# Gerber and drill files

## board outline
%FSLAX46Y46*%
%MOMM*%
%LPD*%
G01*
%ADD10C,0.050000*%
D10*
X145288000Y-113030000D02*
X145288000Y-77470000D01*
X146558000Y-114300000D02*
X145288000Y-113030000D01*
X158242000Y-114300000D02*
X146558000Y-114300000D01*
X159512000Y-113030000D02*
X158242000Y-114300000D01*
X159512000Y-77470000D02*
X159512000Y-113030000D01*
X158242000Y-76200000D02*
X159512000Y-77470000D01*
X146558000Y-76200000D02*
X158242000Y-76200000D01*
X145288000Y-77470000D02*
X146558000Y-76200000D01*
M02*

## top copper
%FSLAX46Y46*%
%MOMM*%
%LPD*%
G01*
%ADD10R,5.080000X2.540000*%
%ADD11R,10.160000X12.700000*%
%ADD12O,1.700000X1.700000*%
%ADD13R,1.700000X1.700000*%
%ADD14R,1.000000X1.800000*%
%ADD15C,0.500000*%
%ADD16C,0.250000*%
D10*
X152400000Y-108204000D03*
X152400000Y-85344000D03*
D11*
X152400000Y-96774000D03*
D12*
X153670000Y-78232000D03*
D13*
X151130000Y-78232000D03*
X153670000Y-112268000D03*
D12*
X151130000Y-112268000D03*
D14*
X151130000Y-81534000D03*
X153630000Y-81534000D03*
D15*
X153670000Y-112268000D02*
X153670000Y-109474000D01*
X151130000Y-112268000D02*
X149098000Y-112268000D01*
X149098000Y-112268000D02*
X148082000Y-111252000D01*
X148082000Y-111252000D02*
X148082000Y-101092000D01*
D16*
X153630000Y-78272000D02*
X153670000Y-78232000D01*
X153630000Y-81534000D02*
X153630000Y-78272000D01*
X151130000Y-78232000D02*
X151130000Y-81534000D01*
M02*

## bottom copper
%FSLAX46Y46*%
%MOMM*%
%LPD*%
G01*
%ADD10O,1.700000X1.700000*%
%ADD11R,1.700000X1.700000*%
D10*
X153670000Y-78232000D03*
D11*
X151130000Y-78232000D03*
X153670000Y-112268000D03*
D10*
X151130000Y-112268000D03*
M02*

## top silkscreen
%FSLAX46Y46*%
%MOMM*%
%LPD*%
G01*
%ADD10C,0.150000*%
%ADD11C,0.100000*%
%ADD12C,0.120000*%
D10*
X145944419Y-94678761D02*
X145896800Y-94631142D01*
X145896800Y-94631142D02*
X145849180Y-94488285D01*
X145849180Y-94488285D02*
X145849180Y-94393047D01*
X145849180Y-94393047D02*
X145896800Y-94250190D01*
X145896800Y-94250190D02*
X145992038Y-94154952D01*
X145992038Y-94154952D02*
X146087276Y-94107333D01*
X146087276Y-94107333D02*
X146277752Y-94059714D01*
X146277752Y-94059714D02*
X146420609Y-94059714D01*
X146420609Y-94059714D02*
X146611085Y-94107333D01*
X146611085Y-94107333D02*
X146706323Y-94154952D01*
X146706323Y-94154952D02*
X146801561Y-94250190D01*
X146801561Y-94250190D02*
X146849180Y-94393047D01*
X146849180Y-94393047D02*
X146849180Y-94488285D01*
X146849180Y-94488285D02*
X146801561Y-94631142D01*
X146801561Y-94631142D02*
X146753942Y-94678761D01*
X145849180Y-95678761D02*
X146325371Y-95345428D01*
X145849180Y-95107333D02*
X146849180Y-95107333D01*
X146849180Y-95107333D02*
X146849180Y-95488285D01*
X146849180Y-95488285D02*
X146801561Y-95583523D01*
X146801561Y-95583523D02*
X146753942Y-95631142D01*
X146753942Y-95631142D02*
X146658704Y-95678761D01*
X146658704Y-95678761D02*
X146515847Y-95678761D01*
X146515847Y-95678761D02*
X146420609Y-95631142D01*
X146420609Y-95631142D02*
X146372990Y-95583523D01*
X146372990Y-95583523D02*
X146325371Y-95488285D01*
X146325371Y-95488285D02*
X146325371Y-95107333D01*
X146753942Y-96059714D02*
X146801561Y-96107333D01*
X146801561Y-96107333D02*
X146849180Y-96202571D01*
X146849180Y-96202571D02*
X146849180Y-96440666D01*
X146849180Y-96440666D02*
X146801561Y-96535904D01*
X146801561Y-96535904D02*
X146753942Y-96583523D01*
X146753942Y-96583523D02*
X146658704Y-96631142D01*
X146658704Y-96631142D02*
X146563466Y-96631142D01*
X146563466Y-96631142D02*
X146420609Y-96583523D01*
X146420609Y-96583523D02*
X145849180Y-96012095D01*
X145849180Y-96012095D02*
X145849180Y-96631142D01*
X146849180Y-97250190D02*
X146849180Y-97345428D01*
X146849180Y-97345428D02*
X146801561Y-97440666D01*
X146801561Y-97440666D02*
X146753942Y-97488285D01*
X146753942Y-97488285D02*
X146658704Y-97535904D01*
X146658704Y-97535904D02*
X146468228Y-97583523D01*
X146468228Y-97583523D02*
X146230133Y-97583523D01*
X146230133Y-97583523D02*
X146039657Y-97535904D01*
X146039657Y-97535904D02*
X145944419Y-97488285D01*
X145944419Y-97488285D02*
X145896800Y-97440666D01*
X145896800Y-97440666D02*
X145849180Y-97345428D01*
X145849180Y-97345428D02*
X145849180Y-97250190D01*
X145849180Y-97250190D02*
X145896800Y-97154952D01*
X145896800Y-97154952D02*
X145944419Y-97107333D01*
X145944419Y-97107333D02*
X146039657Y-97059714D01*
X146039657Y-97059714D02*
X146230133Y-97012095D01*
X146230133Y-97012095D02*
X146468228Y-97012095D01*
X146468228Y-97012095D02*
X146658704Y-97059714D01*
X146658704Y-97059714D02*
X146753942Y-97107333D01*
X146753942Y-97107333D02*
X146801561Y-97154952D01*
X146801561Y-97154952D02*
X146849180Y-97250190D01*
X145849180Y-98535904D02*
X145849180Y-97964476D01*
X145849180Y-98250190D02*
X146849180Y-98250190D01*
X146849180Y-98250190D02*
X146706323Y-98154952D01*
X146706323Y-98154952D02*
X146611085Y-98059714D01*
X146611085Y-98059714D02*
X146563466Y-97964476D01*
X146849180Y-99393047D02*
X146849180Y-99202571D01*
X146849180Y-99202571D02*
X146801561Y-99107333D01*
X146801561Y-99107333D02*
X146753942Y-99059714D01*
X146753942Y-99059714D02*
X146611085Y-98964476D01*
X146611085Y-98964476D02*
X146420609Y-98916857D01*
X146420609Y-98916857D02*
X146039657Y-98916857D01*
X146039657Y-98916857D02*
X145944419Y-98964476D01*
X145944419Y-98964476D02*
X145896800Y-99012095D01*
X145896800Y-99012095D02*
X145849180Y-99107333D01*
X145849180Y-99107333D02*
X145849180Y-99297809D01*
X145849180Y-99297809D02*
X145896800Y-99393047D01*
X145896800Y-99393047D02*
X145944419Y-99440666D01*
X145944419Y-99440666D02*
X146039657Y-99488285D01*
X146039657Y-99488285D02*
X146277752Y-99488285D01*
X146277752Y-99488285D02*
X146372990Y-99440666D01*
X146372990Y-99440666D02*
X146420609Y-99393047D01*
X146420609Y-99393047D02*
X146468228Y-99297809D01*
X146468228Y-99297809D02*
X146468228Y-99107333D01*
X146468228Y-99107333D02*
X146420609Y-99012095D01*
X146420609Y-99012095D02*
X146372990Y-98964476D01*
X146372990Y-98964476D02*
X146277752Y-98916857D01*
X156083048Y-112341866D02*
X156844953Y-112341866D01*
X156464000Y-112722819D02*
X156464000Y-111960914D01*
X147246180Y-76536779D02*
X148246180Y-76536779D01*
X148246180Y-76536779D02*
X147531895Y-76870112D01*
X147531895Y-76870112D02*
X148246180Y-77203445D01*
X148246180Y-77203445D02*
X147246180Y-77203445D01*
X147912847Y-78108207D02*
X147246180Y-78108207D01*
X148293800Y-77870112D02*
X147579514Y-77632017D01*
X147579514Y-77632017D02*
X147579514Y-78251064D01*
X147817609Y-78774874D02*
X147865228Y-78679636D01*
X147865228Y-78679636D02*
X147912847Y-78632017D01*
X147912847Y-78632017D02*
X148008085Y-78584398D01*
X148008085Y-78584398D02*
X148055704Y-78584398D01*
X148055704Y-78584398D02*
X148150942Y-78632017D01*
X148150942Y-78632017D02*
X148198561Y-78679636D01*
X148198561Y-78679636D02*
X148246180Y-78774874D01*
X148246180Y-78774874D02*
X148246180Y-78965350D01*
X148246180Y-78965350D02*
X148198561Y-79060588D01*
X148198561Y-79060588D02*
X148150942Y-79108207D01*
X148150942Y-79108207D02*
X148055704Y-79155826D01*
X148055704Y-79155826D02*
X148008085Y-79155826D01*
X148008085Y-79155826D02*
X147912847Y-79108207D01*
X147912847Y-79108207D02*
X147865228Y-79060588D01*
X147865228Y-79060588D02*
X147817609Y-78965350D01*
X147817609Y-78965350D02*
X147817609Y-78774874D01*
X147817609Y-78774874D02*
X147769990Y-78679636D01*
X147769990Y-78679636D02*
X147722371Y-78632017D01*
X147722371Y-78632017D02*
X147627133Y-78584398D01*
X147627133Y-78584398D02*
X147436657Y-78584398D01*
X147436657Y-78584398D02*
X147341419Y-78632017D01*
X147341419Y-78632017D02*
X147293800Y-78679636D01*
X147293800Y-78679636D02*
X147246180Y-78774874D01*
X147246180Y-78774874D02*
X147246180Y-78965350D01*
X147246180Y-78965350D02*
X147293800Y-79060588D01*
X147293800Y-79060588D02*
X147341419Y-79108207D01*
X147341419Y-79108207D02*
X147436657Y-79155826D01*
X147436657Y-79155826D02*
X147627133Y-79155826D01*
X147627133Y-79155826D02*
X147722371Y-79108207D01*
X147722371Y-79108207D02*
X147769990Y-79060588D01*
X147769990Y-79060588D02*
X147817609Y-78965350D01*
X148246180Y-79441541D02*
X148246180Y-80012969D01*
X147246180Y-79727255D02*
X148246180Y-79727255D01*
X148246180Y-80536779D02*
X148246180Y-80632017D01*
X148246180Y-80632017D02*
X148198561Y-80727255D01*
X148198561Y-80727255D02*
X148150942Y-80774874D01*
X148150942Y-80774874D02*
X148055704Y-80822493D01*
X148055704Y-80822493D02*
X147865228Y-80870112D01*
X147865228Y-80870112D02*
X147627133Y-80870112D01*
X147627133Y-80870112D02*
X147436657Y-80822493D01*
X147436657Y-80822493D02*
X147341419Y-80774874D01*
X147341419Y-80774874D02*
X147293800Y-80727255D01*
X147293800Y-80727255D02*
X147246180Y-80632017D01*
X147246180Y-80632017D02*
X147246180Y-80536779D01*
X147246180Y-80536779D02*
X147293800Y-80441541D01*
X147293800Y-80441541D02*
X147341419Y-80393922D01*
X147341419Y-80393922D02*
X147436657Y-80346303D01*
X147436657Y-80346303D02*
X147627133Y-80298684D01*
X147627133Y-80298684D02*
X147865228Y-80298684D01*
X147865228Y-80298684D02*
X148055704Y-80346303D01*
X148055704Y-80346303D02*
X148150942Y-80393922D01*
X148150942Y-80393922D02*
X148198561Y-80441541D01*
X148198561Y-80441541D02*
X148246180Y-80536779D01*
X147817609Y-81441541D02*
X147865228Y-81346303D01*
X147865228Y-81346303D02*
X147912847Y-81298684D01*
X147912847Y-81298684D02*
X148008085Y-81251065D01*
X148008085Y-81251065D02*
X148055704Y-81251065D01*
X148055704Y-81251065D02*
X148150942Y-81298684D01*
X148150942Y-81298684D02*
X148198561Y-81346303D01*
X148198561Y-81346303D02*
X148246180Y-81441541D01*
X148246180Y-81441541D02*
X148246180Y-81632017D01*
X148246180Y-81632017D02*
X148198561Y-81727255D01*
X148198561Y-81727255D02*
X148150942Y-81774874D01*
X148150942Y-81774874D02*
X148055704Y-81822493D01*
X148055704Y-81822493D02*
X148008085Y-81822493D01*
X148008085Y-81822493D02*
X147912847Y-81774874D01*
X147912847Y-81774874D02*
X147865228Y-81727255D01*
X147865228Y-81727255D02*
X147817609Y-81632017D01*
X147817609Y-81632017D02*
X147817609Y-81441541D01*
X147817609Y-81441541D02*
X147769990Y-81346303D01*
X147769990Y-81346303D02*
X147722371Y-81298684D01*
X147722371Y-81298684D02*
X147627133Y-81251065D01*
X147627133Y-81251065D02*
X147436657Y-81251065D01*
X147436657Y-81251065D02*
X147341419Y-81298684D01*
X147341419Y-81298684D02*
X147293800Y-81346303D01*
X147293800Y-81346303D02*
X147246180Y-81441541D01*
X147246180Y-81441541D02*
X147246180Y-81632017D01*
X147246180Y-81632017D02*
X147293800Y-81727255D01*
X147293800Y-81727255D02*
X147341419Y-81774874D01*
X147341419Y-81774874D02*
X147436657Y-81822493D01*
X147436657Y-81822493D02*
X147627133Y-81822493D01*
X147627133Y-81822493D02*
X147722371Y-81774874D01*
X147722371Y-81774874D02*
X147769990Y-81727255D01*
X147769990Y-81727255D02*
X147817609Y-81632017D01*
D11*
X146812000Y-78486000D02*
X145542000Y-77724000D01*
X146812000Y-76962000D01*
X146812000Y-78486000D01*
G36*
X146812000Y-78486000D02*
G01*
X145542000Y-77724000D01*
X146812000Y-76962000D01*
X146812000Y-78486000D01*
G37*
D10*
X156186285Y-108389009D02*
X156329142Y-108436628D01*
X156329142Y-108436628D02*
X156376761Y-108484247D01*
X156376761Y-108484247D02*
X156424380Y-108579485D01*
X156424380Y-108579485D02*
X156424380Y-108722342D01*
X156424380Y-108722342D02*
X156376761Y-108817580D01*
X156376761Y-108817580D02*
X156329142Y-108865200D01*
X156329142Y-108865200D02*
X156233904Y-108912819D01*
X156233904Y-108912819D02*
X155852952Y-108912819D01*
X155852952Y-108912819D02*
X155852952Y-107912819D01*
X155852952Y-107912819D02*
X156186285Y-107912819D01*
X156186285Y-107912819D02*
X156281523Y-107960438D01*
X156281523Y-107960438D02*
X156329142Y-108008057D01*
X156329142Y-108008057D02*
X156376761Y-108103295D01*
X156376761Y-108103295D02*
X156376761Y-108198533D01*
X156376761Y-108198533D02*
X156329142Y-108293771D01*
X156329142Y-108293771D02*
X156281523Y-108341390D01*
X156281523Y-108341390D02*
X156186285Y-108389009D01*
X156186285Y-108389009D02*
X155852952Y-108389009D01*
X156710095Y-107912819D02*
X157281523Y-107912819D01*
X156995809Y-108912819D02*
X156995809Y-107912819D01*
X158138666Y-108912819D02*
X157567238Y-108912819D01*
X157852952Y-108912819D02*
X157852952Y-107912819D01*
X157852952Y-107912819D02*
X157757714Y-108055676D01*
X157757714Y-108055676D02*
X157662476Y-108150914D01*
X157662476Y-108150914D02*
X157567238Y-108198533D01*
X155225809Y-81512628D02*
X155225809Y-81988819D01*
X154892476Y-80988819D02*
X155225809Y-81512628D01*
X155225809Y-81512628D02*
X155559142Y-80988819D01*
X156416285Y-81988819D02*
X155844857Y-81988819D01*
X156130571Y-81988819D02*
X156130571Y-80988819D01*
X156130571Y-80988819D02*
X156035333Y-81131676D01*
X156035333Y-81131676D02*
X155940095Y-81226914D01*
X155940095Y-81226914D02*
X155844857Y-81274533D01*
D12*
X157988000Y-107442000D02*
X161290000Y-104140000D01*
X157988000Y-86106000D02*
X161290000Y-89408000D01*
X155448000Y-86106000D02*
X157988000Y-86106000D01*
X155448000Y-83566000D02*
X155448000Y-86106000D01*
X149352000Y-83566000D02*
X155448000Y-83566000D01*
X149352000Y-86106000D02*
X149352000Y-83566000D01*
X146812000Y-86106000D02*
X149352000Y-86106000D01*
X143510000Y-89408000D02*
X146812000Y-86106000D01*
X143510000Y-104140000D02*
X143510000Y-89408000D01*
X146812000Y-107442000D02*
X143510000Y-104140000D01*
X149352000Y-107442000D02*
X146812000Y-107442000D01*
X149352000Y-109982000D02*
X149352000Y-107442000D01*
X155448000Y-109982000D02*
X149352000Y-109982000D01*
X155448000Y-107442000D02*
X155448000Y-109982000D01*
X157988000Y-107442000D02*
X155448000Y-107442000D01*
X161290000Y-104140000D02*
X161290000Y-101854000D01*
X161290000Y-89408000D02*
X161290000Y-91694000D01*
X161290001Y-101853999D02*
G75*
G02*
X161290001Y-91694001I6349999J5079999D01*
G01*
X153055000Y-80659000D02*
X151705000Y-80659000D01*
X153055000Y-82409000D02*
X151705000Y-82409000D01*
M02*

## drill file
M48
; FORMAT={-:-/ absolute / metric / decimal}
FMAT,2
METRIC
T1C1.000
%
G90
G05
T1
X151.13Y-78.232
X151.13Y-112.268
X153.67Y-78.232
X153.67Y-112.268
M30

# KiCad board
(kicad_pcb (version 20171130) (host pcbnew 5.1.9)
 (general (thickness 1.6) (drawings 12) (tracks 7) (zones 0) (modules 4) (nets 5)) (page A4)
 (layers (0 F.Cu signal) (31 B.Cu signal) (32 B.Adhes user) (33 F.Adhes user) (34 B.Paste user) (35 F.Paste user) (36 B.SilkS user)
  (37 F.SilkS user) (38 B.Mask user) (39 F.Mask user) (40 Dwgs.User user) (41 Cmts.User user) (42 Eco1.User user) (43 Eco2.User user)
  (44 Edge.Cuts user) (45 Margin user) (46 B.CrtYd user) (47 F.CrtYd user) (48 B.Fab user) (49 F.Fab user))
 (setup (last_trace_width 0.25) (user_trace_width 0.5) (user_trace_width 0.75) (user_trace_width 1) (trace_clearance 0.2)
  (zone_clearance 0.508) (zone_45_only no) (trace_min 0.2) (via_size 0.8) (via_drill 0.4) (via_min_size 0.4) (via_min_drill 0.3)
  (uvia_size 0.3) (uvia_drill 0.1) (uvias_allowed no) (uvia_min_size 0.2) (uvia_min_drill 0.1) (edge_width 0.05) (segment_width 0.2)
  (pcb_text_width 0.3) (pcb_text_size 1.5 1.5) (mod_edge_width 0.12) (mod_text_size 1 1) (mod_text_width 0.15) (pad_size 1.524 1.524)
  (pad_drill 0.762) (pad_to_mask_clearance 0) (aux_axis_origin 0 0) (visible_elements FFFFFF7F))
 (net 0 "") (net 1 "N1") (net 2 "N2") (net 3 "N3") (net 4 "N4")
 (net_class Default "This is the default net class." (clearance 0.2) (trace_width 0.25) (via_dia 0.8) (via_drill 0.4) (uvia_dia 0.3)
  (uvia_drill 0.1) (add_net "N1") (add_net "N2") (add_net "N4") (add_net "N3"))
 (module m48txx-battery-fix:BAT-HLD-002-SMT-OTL (layer F.Cu) (at 152.4 96.774 90)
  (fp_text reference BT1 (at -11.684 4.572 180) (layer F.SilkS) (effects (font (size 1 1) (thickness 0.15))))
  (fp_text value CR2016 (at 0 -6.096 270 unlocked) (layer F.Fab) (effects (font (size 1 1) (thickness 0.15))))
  (fp_line (start -10.668 5.588) (end -7.366 8.89) (layer F.SilkS) (width 0.12))
  (fp_line (start 10.668 5.588) (end 7.366 8.89) (layer F.SilkS) (width 0.12))
  (fp_line (start 10.668 3.048) (end 10.668 5.588) (layer F.SilkS) (width 0.12))
  (fp_line (start 13.208 3.048) (end 10.668 3.048) (layer F.SilkS) (width 0.12))
  (fp_line (start 13.208 -3.048) (end 13.208 3.048) (layer F.SilkS) (width 0.12))
  (fp_line (start 10.668 -3.048) (end 13.208 -3.048) (layer F.SilkS) (width 0.12))
  (fp_line (start 10.668 -5.588) (end 10.668 -3.048) (layer F.SilkS) (width 0.12))
  (fp_line (start 7.366 -8.89) (end 10.668 -5.588) (layer F.SilkS) (width 0.12))
  (fp_line (start -7.366 -8.89) (end 7.366 -8.89) (layer F.SilkS) (width 0.12))
  (fp_line (start -10.668 -5.588) (end -7.366 -8.89) (layer F.SilkS) (width 0.12))
  (fp_line (start -10.668 -3.048) (end -10.668 -5.588) (layer F.SilkS) (width 0.12))
  (fp_line (start -13.208 -3.048) (end -10.668 -3.048) (layer F.SilkS) (width 0.12))
  (fp_line (start -13.208 3.048) (end -13.208 -3.048) (layer F.SilkS) (width 0.12))
  (fp_line (start -10.668 3.048) (end -13.208 3.048) (layer F.SilkS) (width 0.12))
  (fp_line (start -10.668 5.588) (end -10.668 3.048) (layer F.SilkS) (width 0.12))
  (fp_line (start -7.366 8.89) (end -5.08 8.89) (layer F.SilkS) (width 0.12))
  (fp_line (start 7.366 8.89) (end 5.08 8.89) (layer F.SilkS) (width 0.12))
  (fp_arc (start 0 15.24) (end 5.079999 8.890001) (angle -77.31961651) (layer F.SilkS) (width 0.12))
  (pad 1 smd rect (at -12.7 0 90) (size 2.54 5.08) (drill (offset 1.27 0)) (layers F.Cu F.Paste F.Mask) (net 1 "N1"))
  (pad 1 smd rect (at 12.7 0 90) (size 2.54 5.08) (drill (offset -1.27 0)) (layers F.Cu F.Paste F.Mask) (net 1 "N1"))
  (pad 2 smd rect (at 0 0 90) (size 12.7 10.16) (layers F.Cu F.Mask) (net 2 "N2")))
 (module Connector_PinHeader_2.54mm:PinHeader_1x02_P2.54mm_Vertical (layer B.Cu) (at 151.13 78.232 270)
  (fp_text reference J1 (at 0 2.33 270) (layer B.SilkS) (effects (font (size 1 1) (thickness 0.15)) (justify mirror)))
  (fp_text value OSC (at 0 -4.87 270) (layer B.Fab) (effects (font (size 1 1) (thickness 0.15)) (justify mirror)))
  (pad 2 thru_hole oval (at 0 -2.54 270) (size 1.7 1.7) (drill 1) (layers *.Cu *.Mask) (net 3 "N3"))
  (pad 1 thru_hole rect (at 0 0 270) (size 1.7 1.7) (drill 1) (layers *.Cu *.Mask) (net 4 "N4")))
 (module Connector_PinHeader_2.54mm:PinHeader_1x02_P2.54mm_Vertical (layer B.Cu) (at 153.67 112.268 90)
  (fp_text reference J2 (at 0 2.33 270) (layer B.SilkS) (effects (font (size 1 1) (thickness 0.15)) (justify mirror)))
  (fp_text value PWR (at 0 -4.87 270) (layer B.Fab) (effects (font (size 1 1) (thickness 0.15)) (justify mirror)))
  (pad 1 thru_hole rect (at 0 0 90) (size 1.7 1.7) (drill 1) (layers *.Cu *.Mask) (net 1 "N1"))
  (pad 2 thru_hole oval (at 0 -2.54 90) (size 1.7 1.7) (drill 1) (layers *.Cu *.Mask) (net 2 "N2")))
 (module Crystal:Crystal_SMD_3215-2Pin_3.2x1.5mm (layer F.Cu) (at 152.38 81.534 180)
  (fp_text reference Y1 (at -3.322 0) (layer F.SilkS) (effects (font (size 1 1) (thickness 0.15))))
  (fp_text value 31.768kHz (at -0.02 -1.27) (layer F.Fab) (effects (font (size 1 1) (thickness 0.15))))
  (fp_line (start -0.675 0.875) (end 0.675 0.875) (layer F.SilkS) (width 0.12))
  (fp_line (start -0.675 -0.875) (end 0.675 -0.875) (layer F.SilkS) (width 0.12))
  (pad 1 smd rect (at 1.25 0 180) (size 1 1.8) (layers F.Cu F.Paste F.Mask) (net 4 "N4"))
  (pad 2 smd rect (at -1.25 0 180) (size 1 1.8) (layers F.Cu F.Paste F.Mask) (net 3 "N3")))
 (gr_line (start 145.288 113.03) (end 145.288 77.47) (layer Edge.Cuts) (width 0.05))
 (gr_line (start 146.558 114.3) (end 145.288 113.03) (layer Edge.Cuts) (width 0.05))
 (gr_line (start 158.242 114.3) (end 146.558 114.3) (layer Edge.Cuts) (width 0.05))
 (gr_line (start 159.512 113.03) (end 158.242 114.3) (layer Edge.Cuts) (width 0.05))
 (gr_line (start 159.512 77.47) (end 159.512 113.03) (layer Edge.Cuts) (width 0.05))
 (gr_line (start 158.242 76.2) (end 159.512 77.47) (layer Edge.Cuts) (width 0.05))
 (gr_line (start 146.558 76.2) (end 158.242 76.2) (layer Edge.Cuts) (width 0.05))
 (gr_line (start 145.288 77.47) (end 146.558 76.2) (layer Edge.Cuts) (width 0.05))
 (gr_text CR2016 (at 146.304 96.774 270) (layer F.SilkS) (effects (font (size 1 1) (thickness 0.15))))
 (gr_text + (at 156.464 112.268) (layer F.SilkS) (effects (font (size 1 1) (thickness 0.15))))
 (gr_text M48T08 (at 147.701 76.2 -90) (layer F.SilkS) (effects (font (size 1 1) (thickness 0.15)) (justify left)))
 (gr_poly (pts (xy 146.812 78.486) (xy 145.542 77.724) (xy 146.812 76.962)) (layer F.SilkS) (width 0.1))
 (segment (start 153.67 112.268) (end 153.67 109.474) (width 0.5) (layer F.Cu) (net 1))
 (segment (start 151.13 112.268) (end 149.098 112.268) (width 0.5) (layer F.Cu) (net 2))
 (segment (start 149.098 112.268) (end 148.082 111.252) (width 0.5) (layer F.Cu) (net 2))
 (segment (start 148.082 111.252) (end 148.082 101.092) (width 0.5) (layer F.Cu) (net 2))
 (segment (start 153.63 78.272) (end 153.67 78.232) (width 0.25) (layer F.Cu) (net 3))
 (segment (start 153.63 81.534) (end 153.63 78.272) (width 0.25) (layer F.Cu) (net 3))
 (segment (start 151.13 78.232) (end 151.13 81.534) (width 0.25) (layer F.Cu) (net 4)))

